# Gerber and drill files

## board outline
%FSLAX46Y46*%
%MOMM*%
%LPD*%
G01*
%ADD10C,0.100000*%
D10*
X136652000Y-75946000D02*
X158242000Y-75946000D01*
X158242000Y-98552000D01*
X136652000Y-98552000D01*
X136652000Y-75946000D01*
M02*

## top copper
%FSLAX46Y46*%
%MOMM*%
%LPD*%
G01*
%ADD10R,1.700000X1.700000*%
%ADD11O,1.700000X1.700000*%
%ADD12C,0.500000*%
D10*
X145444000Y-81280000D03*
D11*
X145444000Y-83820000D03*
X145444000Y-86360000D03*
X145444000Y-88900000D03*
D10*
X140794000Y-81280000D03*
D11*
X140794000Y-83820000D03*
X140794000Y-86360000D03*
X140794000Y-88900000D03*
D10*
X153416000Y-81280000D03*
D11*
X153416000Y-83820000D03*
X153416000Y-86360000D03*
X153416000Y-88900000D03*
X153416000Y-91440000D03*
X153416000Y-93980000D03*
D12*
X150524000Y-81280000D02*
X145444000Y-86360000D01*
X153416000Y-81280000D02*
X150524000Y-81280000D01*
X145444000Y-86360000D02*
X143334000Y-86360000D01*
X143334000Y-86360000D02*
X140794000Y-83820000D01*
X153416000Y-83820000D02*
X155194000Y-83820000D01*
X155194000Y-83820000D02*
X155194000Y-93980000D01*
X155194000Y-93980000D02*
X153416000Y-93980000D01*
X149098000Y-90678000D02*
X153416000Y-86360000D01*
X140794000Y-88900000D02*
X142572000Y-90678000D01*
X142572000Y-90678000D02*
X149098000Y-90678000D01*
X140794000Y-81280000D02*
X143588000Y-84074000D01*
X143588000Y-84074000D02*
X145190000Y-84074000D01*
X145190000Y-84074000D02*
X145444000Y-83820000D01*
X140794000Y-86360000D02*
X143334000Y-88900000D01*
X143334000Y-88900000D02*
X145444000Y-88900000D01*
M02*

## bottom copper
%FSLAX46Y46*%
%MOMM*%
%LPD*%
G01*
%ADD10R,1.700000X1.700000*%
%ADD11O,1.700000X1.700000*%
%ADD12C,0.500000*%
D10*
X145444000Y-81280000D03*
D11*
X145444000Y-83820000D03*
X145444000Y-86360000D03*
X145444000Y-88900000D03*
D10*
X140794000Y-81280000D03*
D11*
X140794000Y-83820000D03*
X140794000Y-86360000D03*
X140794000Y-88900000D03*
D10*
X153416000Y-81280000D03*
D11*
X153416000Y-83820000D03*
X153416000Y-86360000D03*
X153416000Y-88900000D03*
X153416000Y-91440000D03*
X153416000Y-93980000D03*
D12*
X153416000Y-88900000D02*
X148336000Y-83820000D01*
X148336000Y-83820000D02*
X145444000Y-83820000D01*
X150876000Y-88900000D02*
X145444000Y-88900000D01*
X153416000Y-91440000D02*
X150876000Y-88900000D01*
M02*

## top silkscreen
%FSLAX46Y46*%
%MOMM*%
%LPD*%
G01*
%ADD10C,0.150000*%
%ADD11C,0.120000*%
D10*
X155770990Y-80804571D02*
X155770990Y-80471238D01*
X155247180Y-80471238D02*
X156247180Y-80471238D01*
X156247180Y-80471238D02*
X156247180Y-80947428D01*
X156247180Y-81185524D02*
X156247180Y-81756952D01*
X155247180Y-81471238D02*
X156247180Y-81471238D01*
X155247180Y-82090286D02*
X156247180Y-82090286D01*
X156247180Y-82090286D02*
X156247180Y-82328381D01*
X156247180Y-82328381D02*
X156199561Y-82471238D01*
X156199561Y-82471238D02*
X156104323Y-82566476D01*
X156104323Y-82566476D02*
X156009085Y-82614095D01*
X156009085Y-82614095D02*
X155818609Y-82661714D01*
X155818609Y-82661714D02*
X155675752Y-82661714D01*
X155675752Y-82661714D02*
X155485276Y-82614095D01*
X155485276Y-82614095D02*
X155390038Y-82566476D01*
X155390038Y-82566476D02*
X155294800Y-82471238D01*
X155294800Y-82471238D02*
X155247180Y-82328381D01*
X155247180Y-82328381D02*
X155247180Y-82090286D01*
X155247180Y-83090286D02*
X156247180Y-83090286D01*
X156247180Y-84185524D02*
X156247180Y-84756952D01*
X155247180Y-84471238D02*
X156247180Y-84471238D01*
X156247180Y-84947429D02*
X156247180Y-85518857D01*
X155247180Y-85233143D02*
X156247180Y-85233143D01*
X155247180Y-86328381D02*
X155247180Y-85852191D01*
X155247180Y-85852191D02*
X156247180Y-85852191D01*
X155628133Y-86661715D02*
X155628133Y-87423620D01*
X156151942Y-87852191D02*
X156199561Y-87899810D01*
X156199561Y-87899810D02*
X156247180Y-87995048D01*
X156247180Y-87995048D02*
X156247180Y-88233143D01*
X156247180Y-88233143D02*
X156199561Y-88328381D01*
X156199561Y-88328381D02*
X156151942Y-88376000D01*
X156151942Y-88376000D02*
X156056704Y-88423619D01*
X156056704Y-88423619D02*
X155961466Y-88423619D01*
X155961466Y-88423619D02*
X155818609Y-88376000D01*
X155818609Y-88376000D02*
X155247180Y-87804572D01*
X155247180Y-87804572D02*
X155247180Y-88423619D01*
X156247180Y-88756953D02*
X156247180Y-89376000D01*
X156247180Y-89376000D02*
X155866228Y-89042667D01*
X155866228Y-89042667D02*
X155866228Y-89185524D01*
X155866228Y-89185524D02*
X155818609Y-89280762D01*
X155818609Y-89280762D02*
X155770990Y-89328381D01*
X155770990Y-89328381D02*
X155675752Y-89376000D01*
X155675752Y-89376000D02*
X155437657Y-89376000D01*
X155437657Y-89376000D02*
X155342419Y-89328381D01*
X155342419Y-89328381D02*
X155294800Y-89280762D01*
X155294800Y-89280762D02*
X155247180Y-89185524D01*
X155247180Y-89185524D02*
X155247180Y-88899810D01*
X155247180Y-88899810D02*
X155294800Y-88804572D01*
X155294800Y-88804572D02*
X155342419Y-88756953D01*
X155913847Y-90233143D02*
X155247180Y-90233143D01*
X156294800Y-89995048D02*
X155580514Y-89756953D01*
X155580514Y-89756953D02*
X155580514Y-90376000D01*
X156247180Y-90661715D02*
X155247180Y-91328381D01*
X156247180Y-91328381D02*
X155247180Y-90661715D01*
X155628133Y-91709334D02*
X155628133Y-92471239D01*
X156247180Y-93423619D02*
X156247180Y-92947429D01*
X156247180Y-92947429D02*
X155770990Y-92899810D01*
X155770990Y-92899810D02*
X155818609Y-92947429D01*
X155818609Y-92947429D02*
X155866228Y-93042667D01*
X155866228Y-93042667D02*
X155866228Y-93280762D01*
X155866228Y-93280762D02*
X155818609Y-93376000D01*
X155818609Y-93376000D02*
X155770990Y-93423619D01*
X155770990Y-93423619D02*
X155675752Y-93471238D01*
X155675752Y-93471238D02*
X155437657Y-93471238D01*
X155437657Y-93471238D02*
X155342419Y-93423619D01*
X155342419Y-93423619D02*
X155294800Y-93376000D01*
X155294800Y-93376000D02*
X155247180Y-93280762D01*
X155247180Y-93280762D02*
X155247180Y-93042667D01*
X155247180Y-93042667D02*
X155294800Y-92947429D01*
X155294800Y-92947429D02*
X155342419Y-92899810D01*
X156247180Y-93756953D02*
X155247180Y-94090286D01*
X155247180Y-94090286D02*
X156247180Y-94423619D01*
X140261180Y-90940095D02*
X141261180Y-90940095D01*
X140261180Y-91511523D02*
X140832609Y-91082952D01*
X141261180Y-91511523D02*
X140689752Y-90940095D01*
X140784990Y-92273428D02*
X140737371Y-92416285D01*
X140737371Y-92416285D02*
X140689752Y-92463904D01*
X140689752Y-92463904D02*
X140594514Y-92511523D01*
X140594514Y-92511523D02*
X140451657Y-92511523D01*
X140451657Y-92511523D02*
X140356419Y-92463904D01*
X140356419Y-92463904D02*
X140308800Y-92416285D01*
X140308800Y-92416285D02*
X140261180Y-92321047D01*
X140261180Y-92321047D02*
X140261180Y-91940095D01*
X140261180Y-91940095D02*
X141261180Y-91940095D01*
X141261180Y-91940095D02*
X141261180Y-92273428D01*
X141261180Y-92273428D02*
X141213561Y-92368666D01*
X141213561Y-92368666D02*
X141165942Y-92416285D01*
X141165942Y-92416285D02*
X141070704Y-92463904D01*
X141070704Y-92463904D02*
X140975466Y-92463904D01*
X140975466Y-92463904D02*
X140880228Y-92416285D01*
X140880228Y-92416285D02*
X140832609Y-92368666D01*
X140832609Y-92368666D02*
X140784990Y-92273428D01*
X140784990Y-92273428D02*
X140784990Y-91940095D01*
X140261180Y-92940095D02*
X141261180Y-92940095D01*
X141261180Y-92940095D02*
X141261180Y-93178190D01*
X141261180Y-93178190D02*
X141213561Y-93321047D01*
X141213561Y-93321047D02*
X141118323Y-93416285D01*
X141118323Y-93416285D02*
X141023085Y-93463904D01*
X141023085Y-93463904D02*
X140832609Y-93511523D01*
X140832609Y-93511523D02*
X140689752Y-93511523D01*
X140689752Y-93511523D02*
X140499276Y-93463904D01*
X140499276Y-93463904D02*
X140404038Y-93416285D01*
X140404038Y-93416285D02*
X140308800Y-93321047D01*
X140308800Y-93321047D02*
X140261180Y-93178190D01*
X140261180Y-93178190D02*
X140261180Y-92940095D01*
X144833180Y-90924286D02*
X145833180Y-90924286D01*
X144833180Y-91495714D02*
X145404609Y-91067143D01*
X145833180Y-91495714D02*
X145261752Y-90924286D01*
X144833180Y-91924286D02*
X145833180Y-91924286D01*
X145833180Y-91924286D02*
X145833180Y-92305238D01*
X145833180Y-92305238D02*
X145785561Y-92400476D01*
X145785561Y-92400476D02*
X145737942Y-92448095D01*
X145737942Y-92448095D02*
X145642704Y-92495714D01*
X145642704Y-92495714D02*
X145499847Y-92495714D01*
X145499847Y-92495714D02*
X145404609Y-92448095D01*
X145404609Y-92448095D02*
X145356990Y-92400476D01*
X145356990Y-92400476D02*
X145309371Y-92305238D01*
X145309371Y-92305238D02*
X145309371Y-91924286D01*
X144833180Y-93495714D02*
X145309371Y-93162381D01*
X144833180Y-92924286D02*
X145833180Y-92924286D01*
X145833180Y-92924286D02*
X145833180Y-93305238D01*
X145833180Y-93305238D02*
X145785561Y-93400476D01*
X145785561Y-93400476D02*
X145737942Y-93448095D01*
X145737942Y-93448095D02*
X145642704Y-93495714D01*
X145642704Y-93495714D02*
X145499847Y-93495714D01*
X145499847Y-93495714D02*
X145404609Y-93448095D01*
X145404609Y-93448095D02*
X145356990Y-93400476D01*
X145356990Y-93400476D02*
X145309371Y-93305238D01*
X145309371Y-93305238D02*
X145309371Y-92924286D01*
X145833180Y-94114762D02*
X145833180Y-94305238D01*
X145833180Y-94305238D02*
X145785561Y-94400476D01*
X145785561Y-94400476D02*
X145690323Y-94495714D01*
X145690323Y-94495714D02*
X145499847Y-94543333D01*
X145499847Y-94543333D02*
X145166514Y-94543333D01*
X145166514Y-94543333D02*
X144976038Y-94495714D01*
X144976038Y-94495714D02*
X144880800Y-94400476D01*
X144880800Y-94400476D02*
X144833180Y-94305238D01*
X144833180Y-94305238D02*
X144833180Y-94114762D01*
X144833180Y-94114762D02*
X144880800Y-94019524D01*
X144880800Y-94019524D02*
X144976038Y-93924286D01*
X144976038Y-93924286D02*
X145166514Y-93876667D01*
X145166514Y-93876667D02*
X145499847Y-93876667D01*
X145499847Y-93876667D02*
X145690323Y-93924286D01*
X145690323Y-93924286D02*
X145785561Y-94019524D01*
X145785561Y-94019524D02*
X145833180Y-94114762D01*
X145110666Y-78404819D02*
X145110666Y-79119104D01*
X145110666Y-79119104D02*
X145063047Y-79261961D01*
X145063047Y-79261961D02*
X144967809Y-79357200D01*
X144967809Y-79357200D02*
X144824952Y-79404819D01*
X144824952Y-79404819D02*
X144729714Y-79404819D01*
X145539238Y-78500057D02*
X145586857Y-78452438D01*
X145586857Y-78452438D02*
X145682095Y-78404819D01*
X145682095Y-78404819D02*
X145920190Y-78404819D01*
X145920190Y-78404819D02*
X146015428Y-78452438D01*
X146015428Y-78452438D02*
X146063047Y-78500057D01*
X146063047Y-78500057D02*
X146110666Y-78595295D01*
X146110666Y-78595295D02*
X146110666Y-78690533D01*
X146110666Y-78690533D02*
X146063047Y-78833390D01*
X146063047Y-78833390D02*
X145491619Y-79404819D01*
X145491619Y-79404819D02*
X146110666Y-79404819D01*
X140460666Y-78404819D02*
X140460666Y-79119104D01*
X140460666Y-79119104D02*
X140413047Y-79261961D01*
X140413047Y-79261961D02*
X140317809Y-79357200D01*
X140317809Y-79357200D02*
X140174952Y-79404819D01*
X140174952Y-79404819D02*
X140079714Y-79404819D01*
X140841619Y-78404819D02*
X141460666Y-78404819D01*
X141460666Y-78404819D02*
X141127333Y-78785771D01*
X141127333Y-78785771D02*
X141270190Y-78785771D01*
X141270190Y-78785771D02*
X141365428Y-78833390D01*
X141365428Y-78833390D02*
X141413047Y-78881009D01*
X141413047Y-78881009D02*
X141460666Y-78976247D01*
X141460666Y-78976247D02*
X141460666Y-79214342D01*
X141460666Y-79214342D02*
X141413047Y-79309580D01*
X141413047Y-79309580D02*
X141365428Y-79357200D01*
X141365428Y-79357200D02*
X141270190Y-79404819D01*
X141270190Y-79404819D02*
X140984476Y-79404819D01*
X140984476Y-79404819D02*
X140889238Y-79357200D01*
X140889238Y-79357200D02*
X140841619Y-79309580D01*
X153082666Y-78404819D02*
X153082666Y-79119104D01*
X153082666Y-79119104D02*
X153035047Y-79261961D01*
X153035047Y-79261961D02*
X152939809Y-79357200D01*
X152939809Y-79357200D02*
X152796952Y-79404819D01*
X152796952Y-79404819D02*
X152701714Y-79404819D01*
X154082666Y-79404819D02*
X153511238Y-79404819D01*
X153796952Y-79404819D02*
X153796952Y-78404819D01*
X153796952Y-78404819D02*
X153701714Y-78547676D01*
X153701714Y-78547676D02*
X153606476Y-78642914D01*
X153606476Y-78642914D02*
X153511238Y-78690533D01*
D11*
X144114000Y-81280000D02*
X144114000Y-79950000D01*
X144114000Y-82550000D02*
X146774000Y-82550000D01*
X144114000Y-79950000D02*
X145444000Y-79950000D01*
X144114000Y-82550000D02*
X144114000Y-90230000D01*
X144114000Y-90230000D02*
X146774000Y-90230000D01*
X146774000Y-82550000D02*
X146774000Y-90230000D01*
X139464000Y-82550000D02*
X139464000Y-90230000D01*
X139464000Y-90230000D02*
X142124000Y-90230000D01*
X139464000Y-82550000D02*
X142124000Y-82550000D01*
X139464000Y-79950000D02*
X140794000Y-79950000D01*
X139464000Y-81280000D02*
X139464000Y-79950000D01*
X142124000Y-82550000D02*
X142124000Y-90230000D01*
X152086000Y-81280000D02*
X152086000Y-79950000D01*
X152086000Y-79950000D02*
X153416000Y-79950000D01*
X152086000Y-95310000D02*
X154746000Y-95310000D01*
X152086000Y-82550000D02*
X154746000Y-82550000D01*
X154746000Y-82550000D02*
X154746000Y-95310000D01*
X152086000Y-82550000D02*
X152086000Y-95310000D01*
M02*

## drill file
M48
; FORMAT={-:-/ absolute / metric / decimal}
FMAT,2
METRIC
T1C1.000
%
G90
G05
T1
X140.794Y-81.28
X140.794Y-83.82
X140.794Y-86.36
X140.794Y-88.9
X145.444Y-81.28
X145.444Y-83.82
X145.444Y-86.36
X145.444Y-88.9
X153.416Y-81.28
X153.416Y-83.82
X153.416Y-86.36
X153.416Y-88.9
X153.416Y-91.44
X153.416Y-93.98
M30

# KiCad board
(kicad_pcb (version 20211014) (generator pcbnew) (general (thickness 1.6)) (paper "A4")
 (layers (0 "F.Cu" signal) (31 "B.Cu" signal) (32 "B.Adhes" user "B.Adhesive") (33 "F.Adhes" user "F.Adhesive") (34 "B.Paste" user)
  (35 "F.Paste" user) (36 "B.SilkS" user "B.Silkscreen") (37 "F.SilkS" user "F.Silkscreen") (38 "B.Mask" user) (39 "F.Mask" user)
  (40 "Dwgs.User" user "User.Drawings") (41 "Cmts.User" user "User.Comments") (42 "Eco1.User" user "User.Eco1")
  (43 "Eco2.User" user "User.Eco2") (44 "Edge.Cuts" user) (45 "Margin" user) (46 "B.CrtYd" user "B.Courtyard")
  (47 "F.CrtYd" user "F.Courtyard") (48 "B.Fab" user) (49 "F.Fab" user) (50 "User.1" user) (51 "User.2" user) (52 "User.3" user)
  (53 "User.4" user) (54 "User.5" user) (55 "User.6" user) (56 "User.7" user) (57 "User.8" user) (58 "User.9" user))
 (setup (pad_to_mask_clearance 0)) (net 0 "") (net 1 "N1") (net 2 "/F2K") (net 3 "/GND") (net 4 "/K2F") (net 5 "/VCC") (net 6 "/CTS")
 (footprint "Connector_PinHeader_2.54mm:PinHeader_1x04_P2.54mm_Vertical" (layer "F.Cu") (at 145.444 81.28)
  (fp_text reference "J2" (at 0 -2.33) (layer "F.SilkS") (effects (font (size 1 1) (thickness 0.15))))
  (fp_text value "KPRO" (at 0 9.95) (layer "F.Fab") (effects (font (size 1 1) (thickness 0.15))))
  (fp_line (start -1.33 0) (end -1.33 -1.33) (layer "F.SilkS") (width 0.12))
  (fp_line (start -1.33 1.27) (end 1.33 1.27) (layer "F.SilkS") (width 0.12))
  (fp_line (start -1.33 -1.33) (end 0 -1.33) (layer "F.SilkS") (width 0.12))
  (fp_line (start -1.33 1.27) (end -1.33 8.95) (layer "F.SilkS") (width 0.12))
  (fp_line (start -1.33 8.95) (end 1.33 8.95) (layer "F.SilkS") (width 0.12))
  (fp_line (start 1.33 1.27) (end 1.33 8.95) (layer "F.SilkS") (width 0.12))
  (pad "1" thru_hole rect (at 0 0) (size 1.7 1.7) (drill 1) (layers *.Cu *.Mask) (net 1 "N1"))
  (pad "2" thru_hole oval (at 0 2.54) (size 1.7 1.7) (drill 1) (layers *.Cu *.Mask) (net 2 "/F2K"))
  (pad "3" thru_hole oval (at 0 5.08) (size 1.7 1.7) (drill 1) (layers *.Cu *.Mask) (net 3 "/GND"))
  (pad "4" thru_hole oval (at 0 7.62) (size 1.7 1.7) (drill 1) (layers *.Cu *.Mask) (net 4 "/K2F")))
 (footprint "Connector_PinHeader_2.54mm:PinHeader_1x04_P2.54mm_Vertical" (layer "F.Cu") (at 140.794 81.28)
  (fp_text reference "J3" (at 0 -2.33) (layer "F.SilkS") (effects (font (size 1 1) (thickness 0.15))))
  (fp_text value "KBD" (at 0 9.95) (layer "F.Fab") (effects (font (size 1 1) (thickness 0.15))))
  (fp_line (start -1.33 1.27) (end -1.33 8.95) (layer "F.SilkS") (width 0.12))
  (fp_line (start -1.33 8.95) (end 1.33 8.95) (layer "F.SilkS") (width 0.12))
  (fp_line (start -1.33 1.27) (end 1.33 1.27) (layer "F.SilkS") (width 0.12))
  (fp_line (start -1.33 -1.33) (end 0 -1.33) (layer "F.SilkS") (width 0.12))
  (fp_line (start -1.33 0) (end -1.33 -1.33) (layer "F.SilkS") (width 0.12))
  (fp_line (start 1.33 1.27) (end 1.33 8.95) (layer "F.SilkS") (width 0.12))
  (pad "1" thru_hole rect (at 0 0) (size 1.7 1.7) (drill 1) (layers *.Cu *.Mask) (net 2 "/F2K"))
  (pad "2" thru_hole oval (at 0 2.54) (size 1.7 1.7) (drill 1) (layers *.Cu *.Mask) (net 3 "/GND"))
  (pad "3" thru_hole oval (at 0 5.08) (size 1.7 1.7) (drill 1) (layers *.Cu *.Mask) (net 4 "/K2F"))
  (pad "4" thru_hole oval (at 0 7.62) (size 1.7 1.7) (drill 1) (layers *.Cu *.Mask) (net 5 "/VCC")))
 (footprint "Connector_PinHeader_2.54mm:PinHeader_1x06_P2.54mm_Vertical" (layer "F.Cu") (at 153.416 81.28)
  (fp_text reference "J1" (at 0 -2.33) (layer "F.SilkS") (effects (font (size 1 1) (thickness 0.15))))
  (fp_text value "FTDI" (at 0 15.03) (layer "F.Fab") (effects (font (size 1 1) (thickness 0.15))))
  (fp_line (start -1.33 0) (end -1.33 -1.33) (layer "F.SilkS") (width 0.12))
  (fp_line (start -1.33 -1.33) (end 0 -1.33) (layer "F.SilkS") (width 0.12))
  (fp_line (start -1.33 14.03) (end 1.33 14.03) (layer "F.SilkS") (width 0.12))
  (fp_line (start -1.33 1.27) (end 1.33 1.27) (layer "F.SilkS") (width 0.12))
  (fp_line (start 1.33 1.27) (end 1.33 14.03) (layer "F.SilkS") (width 0.12))
  (fp_line (start -1.33 1.27) (end -1.33 14.03) (layer "F.SilkS") (width 0.12))
  (pad "1" thru_hole rect (at 0 0) (size 1.7 1.7) (drill 1) (layers *.Cu *.Mask) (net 3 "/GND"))
  (pad "2" thru_hole oval (at 0 2.54) (size 1.7 1.7) (drill 1) (layers *.Cu *.Mask) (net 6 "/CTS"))
  (pad "3" thru_hole oval (at 0 5.08) (size 1.7 1.7) (drill 1) (layers *.Cu *.Mask) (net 5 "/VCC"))
  (pad "4" thru_hole oval (at 0 7.62) (size 1.7 1.7) (drill 1) (layers *.Cu *.Mask) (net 2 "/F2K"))
  (pad "5" thru_hole oval (at 0 10.16) (size 1.7 1.7) (drill 1) (layers *.Cu *.Mask) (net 4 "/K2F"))
  (pad "6" thru_hole oval (at 0 12.7) (size 1.7 1.7) (drill 1) (layers *.Cu *.Mask) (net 6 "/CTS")))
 (gr_rect (start 136.652 75.946) (end 158.242 98.552) (layer "Edge.Cuts") (width 0.1) (fill none))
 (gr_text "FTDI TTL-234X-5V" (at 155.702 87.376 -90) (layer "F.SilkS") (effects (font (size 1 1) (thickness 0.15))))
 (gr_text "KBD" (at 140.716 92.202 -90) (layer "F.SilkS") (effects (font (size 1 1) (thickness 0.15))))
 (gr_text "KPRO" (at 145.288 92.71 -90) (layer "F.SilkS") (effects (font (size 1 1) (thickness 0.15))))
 (segment (start 150.524 81.28) (end 145.444 86.36) (width 0.5) (layer "F.Cu") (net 3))
 (segment (start 153.416 81.28) (end 150.524 81.28) (width 0.5) (layer "F.Cu") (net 3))
 (segment (start 145.444 86.36) (end 143.334 86.36) (width 0.5) (layer "F.Cu") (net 3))
 (segment (start 143.334 86.36) (end 140.794 83.82) (width 0.5) (layer "F.Cu") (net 3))
 (segment (start 153.416 83.82) (end 155.194 83.82) (width 0.5) (layer "F.Cu") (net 6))
 (segment (start 155.194 83.82) (end 155.194 93.98) (width 0.5) (layer "F.Cu") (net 6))
 (segment (start 155.194 93.98) (end 153.416 93.98) (width 0.5) (layer "F.Cu") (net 6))
 (segment (start 149.098 90.678) (end 153.416 86.36) (width 0.5) (layer "F.Cu") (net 5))
 (segment (start 140.794 88.9) (end 142.572 90.678) (width 0.5) (layer "F.Cu") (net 5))
 (segment (start 142.572 90.678) (end 149.098 90.678) (width 0.5) (layer "F.Cu") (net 5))
 (segment (start 140.794 81.28) (end 143.588 84.074) (width 0.5) (layer "F.Cu") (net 2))
 (segment (start 143.588 84.074) (end 145.19 84.074) (width 0.5) (layer "F.Cu") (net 2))
 (segment (start 145.19 84.074) (end 145.444 83.82) (width 0.5) (layer "F.Cu") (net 2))
 (segment (start 153.416 88.9) (end 148.336 83.82) (width 0.5) (layer "B.Cu") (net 2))
 (segment (start 148.336 83.82) (end 145.444 83.82) (width 0.5) (layer "B.Cu") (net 2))
 (segment (start 140.794 86.36) (end 143.334 88.9) (width 0.5) (layer "F.Cu") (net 4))
 (segment (start 143.334 88.9) (end 145.444 88.9) (width 0.5) (layer "F.Cu") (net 4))
 (segment (start 150.876 88.9) (end 145.444 88.9) (width 0.5) (layer "B.Cu") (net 4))
 (segment (start 153.416 91.44) (end 150.876 88.9) (width 0.5) (layer "B.Cu") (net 4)))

